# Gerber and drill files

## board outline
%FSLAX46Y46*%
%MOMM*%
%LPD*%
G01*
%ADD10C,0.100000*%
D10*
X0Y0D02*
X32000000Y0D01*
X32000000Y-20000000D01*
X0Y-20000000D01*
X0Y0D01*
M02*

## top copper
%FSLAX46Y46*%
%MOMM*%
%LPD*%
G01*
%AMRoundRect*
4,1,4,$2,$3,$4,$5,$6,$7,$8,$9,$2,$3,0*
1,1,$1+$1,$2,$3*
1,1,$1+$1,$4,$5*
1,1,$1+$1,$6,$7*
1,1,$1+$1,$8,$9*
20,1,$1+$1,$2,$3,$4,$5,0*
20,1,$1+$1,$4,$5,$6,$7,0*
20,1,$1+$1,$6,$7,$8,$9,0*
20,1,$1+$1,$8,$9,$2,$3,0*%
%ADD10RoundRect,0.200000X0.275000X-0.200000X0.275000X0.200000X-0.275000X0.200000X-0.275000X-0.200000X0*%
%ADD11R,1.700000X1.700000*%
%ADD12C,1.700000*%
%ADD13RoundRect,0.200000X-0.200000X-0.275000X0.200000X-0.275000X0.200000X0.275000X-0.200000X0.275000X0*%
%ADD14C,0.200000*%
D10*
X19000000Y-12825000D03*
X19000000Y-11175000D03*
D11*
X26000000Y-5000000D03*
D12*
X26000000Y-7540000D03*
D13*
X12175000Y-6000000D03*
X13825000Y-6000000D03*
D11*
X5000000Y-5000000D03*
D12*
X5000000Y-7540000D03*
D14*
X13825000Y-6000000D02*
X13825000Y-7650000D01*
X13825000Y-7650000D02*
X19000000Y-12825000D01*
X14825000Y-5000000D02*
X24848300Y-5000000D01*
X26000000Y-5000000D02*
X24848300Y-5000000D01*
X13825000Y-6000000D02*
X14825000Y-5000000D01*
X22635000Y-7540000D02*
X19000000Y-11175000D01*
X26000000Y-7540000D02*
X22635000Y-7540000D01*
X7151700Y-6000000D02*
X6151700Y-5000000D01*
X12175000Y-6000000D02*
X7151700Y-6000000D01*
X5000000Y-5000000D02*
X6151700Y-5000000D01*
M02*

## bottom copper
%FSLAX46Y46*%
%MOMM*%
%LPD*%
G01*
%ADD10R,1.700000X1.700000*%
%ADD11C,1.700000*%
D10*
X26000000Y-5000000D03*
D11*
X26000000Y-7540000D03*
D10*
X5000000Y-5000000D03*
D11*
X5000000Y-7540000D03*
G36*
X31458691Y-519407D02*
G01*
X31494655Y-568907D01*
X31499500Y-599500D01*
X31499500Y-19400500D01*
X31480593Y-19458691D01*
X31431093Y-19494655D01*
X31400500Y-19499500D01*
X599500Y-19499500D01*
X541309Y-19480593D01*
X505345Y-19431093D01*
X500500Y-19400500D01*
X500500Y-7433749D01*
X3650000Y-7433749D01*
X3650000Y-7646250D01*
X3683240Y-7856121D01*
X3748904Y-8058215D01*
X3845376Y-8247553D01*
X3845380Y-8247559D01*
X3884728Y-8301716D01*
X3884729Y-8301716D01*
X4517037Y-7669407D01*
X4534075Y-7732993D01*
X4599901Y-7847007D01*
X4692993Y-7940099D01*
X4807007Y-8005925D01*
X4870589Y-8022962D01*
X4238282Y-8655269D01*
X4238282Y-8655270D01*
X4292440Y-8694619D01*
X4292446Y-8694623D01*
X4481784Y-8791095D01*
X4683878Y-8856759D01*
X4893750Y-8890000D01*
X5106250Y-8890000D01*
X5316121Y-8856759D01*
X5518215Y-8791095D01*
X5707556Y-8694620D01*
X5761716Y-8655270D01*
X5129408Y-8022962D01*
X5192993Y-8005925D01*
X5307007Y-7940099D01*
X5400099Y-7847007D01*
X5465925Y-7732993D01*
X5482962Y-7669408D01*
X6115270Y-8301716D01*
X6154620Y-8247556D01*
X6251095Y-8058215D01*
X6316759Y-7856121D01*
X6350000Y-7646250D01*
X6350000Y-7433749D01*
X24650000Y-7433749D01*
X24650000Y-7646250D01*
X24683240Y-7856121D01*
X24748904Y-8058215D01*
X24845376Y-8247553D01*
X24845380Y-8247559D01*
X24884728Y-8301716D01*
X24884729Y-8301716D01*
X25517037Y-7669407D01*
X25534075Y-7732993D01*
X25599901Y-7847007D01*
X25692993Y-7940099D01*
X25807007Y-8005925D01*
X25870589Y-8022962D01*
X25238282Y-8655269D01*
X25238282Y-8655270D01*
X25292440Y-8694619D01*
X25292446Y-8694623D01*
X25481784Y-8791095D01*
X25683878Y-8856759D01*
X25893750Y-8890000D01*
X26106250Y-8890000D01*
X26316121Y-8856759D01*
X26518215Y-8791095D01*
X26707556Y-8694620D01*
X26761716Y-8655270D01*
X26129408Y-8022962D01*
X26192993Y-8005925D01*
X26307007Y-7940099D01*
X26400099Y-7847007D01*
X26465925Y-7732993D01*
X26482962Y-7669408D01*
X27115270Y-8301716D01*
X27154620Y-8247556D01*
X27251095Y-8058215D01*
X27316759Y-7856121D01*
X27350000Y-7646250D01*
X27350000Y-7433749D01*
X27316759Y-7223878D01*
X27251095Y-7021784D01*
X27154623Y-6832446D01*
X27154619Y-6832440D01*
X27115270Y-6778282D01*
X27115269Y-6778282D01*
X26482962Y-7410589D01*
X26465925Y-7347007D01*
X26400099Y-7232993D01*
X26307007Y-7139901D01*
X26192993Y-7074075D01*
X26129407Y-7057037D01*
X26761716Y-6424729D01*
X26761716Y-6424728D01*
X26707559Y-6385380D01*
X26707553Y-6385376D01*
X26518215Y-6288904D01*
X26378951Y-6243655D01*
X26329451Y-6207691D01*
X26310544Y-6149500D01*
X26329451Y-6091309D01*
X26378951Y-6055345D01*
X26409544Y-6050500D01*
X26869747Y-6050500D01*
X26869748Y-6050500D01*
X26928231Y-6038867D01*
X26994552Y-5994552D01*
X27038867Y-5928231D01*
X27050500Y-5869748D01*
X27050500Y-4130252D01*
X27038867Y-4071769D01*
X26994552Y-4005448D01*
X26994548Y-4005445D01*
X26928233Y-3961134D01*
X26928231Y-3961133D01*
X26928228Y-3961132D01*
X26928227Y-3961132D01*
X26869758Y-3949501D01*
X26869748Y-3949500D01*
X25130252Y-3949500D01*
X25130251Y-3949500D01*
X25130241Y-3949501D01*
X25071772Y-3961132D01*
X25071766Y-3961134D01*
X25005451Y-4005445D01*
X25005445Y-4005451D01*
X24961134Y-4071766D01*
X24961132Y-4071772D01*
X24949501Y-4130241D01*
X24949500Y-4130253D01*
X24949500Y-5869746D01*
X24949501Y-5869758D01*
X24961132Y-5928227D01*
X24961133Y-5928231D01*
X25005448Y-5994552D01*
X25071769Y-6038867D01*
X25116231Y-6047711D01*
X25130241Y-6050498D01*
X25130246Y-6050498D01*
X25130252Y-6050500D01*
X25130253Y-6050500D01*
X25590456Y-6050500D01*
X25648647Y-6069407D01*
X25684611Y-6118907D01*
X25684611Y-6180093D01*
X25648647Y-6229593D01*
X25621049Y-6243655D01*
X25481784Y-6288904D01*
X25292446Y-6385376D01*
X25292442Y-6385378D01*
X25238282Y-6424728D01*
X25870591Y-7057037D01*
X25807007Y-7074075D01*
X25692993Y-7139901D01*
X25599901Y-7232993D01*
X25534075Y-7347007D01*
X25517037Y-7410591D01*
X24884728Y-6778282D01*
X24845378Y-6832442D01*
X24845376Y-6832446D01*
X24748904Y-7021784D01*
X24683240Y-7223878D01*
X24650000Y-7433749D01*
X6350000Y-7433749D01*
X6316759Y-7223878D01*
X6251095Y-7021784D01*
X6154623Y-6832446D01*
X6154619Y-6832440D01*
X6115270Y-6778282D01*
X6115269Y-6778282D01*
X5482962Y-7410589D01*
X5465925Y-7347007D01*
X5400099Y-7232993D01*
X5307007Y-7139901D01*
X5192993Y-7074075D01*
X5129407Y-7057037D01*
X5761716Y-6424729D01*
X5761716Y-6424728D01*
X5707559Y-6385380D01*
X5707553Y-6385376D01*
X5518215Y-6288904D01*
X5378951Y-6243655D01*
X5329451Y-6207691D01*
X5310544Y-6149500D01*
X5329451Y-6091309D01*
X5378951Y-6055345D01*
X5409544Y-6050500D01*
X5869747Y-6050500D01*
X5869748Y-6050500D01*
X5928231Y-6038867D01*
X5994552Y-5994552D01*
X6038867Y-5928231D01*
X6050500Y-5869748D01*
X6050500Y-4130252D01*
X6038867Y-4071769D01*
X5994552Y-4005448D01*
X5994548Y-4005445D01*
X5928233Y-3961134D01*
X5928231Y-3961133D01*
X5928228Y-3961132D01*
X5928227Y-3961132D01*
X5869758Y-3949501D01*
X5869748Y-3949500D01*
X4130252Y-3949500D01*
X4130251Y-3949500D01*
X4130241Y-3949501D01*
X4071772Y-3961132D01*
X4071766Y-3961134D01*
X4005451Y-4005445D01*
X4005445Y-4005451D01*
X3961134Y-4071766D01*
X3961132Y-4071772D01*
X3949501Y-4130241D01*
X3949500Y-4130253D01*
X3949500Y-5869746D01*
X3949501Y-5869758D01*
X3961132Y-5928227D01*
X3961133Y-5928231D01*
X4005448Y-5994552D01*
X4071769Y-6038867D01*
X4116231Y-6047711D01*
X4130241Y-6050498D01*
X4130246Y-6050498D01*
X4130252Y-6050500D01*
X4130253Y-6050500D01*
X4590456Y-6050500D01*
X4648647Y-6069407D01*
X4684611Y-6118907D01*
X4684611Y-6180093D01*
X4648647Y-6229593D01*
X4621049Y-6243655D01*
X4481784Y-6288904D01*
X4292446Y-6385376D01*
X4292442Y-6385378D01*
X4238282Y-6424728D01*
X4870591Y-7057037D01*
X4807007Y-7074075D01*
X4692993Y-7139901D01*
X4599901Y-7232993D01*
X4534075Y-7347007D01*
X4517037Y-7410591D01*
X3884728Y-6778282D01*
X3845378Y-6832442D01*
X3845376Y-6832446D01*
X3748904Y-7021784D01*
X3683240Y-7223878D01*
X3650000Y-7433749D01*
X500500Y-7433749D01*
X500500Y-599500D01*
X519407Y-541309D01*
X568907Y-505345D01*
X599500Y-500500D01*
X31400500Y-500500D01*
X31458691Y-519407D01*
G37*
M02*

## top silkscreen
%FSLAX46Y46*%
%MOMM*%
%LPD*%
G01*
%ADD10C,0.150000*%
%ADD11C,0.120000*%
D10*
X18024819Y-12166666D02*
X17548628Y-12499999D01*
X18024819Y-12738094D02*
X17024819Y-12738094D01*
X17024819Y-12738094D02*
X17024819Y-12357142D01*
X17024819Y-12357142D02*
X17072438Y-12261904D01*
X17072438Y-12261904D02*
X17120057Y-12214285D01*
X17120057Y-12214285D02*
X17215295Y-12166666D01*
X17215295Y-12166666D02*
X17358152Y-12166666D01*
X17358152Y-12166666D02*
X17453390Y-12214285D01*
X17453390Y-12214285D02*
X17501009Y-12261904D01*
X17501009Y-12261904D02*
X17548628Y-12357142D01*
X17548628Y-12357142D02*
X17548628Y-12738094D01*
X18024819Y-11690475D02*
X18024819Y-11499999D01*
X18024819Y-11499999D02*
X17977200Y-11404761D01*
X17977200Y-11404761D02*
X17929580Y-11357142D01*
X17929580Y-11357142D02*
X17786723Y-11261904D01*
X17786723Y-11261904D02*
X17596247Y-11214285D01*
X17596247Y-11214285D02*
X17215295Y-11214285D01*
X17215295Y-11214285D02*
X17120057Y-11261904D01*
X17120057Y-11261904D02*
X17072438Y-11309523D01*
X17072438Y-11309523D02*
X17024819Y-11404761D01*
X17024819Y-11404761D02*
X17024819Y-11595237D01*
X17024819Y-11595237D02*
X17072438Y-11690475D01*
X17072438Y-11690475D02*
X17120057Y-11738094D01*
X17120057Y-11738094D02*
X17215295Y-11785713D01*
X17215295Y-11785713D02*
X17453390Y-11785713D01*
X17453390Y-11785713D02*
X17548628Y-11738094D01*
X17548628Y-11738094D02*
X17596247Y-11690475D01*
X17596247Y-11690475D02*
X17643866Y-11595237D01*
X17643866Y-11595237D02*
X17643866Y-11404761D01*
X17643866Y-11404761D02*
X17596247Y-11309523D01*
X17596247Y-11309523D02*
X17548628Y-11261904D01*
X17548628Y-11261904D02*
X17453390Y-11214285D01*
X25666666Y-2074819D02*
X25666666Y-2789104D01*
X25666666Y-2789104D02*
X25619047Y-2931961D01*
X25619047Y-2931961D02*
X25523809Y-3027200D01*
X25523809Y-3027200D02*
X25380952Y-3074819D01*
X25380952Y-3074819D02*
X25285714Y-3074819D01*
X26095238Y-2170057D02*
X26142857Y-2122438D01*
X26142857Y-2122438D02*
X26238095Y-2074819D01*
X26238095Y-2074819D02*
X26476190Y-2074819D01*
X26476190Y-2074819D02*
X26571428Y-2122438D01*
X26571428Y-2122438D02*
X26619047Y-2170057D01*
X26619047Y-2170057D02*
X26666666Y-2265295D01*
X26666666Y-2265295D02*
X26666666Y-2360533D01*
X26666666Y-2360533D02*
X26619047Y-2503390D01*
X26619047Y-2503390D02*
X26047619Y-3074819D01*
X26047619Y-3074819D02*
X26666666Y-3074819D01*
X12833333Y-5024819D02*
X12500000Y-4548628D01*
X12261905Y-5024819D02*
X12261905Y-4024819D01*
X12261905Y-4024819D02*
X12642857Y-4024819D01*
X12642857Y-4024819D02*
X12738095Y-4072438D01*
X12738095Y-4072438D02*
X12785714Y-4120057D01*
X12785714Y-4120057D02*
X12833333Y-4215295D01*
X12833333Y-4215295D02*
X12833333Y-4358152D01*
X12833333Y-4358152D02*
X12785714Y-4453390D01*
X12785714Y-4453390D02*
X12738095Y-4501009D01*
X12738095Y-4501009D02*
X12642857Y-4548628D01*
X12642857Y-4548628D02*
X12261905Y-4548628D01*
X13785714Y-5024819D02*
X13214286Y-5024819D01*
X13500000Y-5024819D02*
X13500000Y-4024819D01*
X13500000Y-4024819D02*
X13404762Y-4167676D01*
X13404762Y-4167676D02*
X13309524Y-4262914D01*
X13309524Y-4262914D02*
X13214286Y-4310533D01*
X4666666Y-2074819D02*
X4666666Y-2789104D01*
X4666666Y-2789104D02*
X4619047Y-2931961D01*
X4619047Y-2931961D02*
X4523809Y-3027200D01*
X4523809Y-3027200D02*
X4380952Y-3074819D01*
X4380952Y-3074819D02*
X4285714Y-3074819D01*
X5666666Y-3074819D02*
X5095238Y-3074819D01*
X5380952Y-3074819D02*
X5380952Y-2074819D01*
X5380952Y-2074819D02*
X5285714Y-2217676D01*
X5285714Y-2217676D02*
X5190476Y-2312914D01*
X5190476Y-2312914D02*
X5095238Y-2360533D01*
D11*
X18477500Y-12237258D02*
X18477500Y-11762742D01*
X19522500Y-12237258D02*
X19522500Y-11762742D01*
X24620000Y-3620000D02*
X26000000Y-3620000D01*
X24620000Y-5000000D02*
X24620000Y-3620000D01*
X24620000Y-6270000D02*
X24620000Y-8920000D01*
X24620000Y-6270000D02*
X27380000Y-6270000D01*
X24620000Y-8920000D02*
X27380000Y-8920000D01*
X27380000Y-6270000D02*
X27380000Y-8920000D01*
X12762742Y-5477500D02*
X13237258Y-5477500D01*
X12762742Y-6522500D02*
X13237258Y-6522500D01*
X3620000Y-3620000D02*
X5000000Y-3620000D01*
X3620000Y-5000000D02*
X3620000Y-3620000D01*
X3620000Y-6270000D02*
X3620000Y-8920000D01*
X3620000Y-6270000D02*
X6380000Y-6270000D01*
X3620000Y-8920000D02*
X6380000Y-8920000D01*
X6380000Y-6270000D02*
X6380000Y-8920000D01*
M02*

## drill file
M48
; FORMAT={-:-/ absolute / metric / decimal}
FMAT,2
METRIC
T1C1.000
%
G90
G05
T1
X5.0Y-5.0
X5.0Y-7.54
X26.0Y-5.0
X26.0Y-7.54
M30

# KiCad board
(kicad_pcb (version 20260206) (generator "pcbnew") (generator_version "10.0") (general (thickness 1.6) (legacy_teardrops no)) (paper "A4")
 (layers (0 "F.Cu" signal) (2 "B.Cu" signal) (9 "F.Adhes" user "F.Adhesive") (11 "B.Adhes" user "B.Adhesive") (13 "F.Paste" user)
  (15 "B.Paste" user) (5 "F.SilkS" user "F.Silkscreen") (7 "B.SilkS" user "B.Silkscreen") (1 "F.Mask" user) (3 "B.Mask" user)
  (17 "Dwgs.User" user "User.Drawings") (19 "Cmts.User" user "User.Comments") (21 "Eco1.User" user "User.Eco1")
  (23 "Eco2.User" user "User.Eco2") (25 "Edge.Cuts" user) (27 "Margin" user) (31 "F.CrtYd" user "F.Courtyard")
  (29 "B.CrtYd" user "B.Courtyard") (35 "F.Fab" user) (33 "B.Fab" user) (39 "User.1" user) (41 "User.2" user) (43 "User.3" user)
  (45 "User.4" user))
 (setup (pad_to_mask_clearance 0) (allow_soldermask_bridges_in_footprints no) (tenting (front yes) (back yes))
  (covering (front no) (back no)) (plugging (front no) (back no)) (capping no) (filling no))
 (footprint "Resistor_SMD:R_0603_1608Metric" (layer "F.Cu") (at 19 12 90)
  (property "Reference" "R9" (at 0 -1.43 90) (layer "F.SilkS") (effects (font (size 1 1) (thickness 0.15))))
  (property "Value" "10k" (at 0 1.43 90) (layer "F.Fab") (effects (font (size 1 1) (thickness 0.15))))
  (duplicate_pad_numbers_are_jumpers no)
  (fp_line (start -0.237258 -0.5225) (end 0.237258 -0.5225) (stroke (width 0.12) (type solid)) (layer "F.SilkS"))
  (fp_line (start -0.237258 0.5225) (end 0.237258 0.5225) (stroke (width 0.12) (type solid)) (layer "F.SilkS"))
  (pad "1" smd roundrect (at -0.825 0 90) (size 0.8 0.95) (layers "F.Cu" "F.Mask" "F.Paste") (roundrect_rratio 0.25) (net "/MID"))
  (pad "2" smd roundrect (at 0.825 0 90) (size 0.8 0.95) (layers "F.Cu" "F.Mask" "F.Paste") (roundrect_rratio 0.25) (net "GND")))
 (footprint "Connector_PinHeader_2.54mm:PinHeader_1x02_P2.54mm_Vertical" (layer "F.Cu") (at 26 5)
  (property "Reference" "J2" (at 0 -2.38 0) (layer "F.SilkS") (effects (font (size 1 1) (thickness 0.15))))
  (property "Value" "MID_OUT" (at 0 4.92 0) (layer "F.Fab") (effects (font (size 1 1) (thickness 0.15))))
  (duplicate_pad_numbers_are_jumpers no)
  (fp_line (start -1.38 -1.38) (end 0 -1.38) (stroke (width 0.12) (type solid)) (layer "F.SilkS"))
  (fp_line (start -1.38 0) (end -1.38 -1.38) (stroke (width 0.12) (type solid)) (layer "F.SilkS"))
  (fp_line (start -1.38 1.27) (end -1.38 3.92) (stroke (width 0.12) (type solid)) (layer "F.SilkS"))
  (fp_line (start -1.38 1.27) (end 1.38 1.27) (stroke (width 0.12) (type solid)) (layer "F.SilkS"))
  (fp_line (start -1.38 3.92) (end 1.38 3.92) (stroke (width 0.12) (type solid)) (layer "F.SilkS"))
  (fp_line (start 1.38 1.27) (end 1.38 3.92) (stroke (width 0.12) (type solid)) (layer "F.SilkS"))
  (pad "1" thru_hole rect (at 0 0) (size 1.7 1.7) (drill 1) (layers "*.Cu" "*.Mask") (remove_unused_layers no) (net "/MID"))
  (pad "2" thru_hole circle (at 0 2.54) (size 1.7 1.7) (drill 1) (layers "*.Cu" "*.Mask") (remove_unused_layers no) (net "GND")))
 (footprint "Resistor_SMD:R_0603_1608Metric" (layer "F.Cu") (at 13 6)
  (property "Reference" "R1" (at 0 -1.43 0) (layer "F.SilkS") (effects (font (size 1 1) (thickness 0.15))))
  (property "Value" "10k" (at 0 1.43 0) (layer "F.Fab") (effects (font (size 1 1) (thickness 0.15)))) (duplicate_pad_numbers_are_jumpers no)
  (fp_line (start -0.237258 -0.5225) (end 0.237258 -0.5225) (stroke (width 0.12) (type solid)) (layer "F.SilkS"))
  (fp_line (start -0.237258 0.5225) (end 0.237258 0.5225) (stroke (width 0.12) (type solid)) (layer "F.SilkS"))
  (pad "1" smd roundrect (at -0.825 0) (size 0.8 0.95) (layers "F.Cu" "F.Mask" "F.Paste") (roundrect_rratio 0.25) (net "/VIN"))
  (pad "2" smd roundrect (at 0.825 0) (size 0.8 0.95) (layers "F.Cu" "F.Mask" "F.Paste") (roundrect_rratio 0.25) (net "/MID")))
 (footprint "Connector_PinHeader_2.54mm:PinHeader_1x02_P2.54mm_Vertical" (layer "F.Cu") (at 5 5)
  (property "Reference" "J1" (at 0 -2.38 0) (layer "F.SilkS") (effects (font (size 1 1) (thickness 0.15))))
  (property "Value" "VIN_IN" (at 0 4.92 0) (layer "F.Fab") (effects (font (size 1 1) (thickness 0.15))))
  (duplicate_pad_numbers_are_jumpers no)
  (fp_line (start -1.38 -1.38) (end 0 -1.38) (stroke (width 0.12) (type solid)) (layer "F.SilkS"))
  (fp_line (start -1.38 0) (end -1.38 -1.38) (stroke (width 0.12) (type solid)) (layer "F.SilkS"))
  (fp_line (start -1.38 1.27) (end -1.38 3.92) (stroke (width 0.12) (type solid)) (layer "F.SilkS"))
  (fp_line (start -1.38 1.27) (end 1.38 1.27) (stroke (width 0.12) (type solid)) (layer "F.SilkS"))
  (fp_line (start -1.38 3.92) (end 1.38 3.92) (stroke (width 0.12) (type solid)) (layer "F.SilkS"))
  (fp_line (start 1.38 1.27) (end 1.38 3.92) (stroke (width 0.12) (type solid)) (layer "F.SilkS"))
  (pad "1" thru_hole rect (at 0 0) (size 1.7 1.7) (drill 1) (layers "*.Cu" "*.Mask") (remove_unused_layers no) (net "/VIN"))
  (pad "2" thru_hole circle (at 0 2.54) (size 1.7 1.7) (drill 1) (layers "*.Cu" "*.Mask") (remove_unused_layers no) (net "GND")))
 (gr_rect (start 0 0) (end 32 20) (stroke (width 0.1) (type default)) (fill no) (layer "Edge.Cuts"))
 (segment (start 13.825 6) (end 13.825 7.65) (width 0.2) (layer "F.Cu") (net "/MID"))
 (segment (start 13.825 7.65) (end 19 12.825) (width 0.2) (layer "F.Cu") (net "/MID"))
 (segment (start 14.825 5) (end 24.8483 5) (width 0.2) (layer "F.Cu") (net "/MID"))
 (segment (start 26 5) (end 24.8483 5) (width 0.2) (layer "F.Cu") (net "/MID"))
 (segment (start 13.825 6) (end 14.825 5) (width 0.2) (layer "F.Cu") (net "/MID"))
 (segment (start 22.635 7.54) (end 19 11.175) (width 0.2) (layer "F.Cu") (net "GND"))
 (segment (start 26 7.54) (end 22.635 7.54) (width 0.2) (layer "F.Cu") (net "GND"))
 (segment (start 7.1517 6) (end 6.1517 5) (width 0.2) (layer "F.Cu") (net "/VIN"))
 (segment (start 12.175 6) (end 7.1517 6) (width 0.2) (layer "F.Cu") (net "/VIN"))
 (segment (start 5 5) (end 6.1517 5) (width 0.2) (layer "F.Cu") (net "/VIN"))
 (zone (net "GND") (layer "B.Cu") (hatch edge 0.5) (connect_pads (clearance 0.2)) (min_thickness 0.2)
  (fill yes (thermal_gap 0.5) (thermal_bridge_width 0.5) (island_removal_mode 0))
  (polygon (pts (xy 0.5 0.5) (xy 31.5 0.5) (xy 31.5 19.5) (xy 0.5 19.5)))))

